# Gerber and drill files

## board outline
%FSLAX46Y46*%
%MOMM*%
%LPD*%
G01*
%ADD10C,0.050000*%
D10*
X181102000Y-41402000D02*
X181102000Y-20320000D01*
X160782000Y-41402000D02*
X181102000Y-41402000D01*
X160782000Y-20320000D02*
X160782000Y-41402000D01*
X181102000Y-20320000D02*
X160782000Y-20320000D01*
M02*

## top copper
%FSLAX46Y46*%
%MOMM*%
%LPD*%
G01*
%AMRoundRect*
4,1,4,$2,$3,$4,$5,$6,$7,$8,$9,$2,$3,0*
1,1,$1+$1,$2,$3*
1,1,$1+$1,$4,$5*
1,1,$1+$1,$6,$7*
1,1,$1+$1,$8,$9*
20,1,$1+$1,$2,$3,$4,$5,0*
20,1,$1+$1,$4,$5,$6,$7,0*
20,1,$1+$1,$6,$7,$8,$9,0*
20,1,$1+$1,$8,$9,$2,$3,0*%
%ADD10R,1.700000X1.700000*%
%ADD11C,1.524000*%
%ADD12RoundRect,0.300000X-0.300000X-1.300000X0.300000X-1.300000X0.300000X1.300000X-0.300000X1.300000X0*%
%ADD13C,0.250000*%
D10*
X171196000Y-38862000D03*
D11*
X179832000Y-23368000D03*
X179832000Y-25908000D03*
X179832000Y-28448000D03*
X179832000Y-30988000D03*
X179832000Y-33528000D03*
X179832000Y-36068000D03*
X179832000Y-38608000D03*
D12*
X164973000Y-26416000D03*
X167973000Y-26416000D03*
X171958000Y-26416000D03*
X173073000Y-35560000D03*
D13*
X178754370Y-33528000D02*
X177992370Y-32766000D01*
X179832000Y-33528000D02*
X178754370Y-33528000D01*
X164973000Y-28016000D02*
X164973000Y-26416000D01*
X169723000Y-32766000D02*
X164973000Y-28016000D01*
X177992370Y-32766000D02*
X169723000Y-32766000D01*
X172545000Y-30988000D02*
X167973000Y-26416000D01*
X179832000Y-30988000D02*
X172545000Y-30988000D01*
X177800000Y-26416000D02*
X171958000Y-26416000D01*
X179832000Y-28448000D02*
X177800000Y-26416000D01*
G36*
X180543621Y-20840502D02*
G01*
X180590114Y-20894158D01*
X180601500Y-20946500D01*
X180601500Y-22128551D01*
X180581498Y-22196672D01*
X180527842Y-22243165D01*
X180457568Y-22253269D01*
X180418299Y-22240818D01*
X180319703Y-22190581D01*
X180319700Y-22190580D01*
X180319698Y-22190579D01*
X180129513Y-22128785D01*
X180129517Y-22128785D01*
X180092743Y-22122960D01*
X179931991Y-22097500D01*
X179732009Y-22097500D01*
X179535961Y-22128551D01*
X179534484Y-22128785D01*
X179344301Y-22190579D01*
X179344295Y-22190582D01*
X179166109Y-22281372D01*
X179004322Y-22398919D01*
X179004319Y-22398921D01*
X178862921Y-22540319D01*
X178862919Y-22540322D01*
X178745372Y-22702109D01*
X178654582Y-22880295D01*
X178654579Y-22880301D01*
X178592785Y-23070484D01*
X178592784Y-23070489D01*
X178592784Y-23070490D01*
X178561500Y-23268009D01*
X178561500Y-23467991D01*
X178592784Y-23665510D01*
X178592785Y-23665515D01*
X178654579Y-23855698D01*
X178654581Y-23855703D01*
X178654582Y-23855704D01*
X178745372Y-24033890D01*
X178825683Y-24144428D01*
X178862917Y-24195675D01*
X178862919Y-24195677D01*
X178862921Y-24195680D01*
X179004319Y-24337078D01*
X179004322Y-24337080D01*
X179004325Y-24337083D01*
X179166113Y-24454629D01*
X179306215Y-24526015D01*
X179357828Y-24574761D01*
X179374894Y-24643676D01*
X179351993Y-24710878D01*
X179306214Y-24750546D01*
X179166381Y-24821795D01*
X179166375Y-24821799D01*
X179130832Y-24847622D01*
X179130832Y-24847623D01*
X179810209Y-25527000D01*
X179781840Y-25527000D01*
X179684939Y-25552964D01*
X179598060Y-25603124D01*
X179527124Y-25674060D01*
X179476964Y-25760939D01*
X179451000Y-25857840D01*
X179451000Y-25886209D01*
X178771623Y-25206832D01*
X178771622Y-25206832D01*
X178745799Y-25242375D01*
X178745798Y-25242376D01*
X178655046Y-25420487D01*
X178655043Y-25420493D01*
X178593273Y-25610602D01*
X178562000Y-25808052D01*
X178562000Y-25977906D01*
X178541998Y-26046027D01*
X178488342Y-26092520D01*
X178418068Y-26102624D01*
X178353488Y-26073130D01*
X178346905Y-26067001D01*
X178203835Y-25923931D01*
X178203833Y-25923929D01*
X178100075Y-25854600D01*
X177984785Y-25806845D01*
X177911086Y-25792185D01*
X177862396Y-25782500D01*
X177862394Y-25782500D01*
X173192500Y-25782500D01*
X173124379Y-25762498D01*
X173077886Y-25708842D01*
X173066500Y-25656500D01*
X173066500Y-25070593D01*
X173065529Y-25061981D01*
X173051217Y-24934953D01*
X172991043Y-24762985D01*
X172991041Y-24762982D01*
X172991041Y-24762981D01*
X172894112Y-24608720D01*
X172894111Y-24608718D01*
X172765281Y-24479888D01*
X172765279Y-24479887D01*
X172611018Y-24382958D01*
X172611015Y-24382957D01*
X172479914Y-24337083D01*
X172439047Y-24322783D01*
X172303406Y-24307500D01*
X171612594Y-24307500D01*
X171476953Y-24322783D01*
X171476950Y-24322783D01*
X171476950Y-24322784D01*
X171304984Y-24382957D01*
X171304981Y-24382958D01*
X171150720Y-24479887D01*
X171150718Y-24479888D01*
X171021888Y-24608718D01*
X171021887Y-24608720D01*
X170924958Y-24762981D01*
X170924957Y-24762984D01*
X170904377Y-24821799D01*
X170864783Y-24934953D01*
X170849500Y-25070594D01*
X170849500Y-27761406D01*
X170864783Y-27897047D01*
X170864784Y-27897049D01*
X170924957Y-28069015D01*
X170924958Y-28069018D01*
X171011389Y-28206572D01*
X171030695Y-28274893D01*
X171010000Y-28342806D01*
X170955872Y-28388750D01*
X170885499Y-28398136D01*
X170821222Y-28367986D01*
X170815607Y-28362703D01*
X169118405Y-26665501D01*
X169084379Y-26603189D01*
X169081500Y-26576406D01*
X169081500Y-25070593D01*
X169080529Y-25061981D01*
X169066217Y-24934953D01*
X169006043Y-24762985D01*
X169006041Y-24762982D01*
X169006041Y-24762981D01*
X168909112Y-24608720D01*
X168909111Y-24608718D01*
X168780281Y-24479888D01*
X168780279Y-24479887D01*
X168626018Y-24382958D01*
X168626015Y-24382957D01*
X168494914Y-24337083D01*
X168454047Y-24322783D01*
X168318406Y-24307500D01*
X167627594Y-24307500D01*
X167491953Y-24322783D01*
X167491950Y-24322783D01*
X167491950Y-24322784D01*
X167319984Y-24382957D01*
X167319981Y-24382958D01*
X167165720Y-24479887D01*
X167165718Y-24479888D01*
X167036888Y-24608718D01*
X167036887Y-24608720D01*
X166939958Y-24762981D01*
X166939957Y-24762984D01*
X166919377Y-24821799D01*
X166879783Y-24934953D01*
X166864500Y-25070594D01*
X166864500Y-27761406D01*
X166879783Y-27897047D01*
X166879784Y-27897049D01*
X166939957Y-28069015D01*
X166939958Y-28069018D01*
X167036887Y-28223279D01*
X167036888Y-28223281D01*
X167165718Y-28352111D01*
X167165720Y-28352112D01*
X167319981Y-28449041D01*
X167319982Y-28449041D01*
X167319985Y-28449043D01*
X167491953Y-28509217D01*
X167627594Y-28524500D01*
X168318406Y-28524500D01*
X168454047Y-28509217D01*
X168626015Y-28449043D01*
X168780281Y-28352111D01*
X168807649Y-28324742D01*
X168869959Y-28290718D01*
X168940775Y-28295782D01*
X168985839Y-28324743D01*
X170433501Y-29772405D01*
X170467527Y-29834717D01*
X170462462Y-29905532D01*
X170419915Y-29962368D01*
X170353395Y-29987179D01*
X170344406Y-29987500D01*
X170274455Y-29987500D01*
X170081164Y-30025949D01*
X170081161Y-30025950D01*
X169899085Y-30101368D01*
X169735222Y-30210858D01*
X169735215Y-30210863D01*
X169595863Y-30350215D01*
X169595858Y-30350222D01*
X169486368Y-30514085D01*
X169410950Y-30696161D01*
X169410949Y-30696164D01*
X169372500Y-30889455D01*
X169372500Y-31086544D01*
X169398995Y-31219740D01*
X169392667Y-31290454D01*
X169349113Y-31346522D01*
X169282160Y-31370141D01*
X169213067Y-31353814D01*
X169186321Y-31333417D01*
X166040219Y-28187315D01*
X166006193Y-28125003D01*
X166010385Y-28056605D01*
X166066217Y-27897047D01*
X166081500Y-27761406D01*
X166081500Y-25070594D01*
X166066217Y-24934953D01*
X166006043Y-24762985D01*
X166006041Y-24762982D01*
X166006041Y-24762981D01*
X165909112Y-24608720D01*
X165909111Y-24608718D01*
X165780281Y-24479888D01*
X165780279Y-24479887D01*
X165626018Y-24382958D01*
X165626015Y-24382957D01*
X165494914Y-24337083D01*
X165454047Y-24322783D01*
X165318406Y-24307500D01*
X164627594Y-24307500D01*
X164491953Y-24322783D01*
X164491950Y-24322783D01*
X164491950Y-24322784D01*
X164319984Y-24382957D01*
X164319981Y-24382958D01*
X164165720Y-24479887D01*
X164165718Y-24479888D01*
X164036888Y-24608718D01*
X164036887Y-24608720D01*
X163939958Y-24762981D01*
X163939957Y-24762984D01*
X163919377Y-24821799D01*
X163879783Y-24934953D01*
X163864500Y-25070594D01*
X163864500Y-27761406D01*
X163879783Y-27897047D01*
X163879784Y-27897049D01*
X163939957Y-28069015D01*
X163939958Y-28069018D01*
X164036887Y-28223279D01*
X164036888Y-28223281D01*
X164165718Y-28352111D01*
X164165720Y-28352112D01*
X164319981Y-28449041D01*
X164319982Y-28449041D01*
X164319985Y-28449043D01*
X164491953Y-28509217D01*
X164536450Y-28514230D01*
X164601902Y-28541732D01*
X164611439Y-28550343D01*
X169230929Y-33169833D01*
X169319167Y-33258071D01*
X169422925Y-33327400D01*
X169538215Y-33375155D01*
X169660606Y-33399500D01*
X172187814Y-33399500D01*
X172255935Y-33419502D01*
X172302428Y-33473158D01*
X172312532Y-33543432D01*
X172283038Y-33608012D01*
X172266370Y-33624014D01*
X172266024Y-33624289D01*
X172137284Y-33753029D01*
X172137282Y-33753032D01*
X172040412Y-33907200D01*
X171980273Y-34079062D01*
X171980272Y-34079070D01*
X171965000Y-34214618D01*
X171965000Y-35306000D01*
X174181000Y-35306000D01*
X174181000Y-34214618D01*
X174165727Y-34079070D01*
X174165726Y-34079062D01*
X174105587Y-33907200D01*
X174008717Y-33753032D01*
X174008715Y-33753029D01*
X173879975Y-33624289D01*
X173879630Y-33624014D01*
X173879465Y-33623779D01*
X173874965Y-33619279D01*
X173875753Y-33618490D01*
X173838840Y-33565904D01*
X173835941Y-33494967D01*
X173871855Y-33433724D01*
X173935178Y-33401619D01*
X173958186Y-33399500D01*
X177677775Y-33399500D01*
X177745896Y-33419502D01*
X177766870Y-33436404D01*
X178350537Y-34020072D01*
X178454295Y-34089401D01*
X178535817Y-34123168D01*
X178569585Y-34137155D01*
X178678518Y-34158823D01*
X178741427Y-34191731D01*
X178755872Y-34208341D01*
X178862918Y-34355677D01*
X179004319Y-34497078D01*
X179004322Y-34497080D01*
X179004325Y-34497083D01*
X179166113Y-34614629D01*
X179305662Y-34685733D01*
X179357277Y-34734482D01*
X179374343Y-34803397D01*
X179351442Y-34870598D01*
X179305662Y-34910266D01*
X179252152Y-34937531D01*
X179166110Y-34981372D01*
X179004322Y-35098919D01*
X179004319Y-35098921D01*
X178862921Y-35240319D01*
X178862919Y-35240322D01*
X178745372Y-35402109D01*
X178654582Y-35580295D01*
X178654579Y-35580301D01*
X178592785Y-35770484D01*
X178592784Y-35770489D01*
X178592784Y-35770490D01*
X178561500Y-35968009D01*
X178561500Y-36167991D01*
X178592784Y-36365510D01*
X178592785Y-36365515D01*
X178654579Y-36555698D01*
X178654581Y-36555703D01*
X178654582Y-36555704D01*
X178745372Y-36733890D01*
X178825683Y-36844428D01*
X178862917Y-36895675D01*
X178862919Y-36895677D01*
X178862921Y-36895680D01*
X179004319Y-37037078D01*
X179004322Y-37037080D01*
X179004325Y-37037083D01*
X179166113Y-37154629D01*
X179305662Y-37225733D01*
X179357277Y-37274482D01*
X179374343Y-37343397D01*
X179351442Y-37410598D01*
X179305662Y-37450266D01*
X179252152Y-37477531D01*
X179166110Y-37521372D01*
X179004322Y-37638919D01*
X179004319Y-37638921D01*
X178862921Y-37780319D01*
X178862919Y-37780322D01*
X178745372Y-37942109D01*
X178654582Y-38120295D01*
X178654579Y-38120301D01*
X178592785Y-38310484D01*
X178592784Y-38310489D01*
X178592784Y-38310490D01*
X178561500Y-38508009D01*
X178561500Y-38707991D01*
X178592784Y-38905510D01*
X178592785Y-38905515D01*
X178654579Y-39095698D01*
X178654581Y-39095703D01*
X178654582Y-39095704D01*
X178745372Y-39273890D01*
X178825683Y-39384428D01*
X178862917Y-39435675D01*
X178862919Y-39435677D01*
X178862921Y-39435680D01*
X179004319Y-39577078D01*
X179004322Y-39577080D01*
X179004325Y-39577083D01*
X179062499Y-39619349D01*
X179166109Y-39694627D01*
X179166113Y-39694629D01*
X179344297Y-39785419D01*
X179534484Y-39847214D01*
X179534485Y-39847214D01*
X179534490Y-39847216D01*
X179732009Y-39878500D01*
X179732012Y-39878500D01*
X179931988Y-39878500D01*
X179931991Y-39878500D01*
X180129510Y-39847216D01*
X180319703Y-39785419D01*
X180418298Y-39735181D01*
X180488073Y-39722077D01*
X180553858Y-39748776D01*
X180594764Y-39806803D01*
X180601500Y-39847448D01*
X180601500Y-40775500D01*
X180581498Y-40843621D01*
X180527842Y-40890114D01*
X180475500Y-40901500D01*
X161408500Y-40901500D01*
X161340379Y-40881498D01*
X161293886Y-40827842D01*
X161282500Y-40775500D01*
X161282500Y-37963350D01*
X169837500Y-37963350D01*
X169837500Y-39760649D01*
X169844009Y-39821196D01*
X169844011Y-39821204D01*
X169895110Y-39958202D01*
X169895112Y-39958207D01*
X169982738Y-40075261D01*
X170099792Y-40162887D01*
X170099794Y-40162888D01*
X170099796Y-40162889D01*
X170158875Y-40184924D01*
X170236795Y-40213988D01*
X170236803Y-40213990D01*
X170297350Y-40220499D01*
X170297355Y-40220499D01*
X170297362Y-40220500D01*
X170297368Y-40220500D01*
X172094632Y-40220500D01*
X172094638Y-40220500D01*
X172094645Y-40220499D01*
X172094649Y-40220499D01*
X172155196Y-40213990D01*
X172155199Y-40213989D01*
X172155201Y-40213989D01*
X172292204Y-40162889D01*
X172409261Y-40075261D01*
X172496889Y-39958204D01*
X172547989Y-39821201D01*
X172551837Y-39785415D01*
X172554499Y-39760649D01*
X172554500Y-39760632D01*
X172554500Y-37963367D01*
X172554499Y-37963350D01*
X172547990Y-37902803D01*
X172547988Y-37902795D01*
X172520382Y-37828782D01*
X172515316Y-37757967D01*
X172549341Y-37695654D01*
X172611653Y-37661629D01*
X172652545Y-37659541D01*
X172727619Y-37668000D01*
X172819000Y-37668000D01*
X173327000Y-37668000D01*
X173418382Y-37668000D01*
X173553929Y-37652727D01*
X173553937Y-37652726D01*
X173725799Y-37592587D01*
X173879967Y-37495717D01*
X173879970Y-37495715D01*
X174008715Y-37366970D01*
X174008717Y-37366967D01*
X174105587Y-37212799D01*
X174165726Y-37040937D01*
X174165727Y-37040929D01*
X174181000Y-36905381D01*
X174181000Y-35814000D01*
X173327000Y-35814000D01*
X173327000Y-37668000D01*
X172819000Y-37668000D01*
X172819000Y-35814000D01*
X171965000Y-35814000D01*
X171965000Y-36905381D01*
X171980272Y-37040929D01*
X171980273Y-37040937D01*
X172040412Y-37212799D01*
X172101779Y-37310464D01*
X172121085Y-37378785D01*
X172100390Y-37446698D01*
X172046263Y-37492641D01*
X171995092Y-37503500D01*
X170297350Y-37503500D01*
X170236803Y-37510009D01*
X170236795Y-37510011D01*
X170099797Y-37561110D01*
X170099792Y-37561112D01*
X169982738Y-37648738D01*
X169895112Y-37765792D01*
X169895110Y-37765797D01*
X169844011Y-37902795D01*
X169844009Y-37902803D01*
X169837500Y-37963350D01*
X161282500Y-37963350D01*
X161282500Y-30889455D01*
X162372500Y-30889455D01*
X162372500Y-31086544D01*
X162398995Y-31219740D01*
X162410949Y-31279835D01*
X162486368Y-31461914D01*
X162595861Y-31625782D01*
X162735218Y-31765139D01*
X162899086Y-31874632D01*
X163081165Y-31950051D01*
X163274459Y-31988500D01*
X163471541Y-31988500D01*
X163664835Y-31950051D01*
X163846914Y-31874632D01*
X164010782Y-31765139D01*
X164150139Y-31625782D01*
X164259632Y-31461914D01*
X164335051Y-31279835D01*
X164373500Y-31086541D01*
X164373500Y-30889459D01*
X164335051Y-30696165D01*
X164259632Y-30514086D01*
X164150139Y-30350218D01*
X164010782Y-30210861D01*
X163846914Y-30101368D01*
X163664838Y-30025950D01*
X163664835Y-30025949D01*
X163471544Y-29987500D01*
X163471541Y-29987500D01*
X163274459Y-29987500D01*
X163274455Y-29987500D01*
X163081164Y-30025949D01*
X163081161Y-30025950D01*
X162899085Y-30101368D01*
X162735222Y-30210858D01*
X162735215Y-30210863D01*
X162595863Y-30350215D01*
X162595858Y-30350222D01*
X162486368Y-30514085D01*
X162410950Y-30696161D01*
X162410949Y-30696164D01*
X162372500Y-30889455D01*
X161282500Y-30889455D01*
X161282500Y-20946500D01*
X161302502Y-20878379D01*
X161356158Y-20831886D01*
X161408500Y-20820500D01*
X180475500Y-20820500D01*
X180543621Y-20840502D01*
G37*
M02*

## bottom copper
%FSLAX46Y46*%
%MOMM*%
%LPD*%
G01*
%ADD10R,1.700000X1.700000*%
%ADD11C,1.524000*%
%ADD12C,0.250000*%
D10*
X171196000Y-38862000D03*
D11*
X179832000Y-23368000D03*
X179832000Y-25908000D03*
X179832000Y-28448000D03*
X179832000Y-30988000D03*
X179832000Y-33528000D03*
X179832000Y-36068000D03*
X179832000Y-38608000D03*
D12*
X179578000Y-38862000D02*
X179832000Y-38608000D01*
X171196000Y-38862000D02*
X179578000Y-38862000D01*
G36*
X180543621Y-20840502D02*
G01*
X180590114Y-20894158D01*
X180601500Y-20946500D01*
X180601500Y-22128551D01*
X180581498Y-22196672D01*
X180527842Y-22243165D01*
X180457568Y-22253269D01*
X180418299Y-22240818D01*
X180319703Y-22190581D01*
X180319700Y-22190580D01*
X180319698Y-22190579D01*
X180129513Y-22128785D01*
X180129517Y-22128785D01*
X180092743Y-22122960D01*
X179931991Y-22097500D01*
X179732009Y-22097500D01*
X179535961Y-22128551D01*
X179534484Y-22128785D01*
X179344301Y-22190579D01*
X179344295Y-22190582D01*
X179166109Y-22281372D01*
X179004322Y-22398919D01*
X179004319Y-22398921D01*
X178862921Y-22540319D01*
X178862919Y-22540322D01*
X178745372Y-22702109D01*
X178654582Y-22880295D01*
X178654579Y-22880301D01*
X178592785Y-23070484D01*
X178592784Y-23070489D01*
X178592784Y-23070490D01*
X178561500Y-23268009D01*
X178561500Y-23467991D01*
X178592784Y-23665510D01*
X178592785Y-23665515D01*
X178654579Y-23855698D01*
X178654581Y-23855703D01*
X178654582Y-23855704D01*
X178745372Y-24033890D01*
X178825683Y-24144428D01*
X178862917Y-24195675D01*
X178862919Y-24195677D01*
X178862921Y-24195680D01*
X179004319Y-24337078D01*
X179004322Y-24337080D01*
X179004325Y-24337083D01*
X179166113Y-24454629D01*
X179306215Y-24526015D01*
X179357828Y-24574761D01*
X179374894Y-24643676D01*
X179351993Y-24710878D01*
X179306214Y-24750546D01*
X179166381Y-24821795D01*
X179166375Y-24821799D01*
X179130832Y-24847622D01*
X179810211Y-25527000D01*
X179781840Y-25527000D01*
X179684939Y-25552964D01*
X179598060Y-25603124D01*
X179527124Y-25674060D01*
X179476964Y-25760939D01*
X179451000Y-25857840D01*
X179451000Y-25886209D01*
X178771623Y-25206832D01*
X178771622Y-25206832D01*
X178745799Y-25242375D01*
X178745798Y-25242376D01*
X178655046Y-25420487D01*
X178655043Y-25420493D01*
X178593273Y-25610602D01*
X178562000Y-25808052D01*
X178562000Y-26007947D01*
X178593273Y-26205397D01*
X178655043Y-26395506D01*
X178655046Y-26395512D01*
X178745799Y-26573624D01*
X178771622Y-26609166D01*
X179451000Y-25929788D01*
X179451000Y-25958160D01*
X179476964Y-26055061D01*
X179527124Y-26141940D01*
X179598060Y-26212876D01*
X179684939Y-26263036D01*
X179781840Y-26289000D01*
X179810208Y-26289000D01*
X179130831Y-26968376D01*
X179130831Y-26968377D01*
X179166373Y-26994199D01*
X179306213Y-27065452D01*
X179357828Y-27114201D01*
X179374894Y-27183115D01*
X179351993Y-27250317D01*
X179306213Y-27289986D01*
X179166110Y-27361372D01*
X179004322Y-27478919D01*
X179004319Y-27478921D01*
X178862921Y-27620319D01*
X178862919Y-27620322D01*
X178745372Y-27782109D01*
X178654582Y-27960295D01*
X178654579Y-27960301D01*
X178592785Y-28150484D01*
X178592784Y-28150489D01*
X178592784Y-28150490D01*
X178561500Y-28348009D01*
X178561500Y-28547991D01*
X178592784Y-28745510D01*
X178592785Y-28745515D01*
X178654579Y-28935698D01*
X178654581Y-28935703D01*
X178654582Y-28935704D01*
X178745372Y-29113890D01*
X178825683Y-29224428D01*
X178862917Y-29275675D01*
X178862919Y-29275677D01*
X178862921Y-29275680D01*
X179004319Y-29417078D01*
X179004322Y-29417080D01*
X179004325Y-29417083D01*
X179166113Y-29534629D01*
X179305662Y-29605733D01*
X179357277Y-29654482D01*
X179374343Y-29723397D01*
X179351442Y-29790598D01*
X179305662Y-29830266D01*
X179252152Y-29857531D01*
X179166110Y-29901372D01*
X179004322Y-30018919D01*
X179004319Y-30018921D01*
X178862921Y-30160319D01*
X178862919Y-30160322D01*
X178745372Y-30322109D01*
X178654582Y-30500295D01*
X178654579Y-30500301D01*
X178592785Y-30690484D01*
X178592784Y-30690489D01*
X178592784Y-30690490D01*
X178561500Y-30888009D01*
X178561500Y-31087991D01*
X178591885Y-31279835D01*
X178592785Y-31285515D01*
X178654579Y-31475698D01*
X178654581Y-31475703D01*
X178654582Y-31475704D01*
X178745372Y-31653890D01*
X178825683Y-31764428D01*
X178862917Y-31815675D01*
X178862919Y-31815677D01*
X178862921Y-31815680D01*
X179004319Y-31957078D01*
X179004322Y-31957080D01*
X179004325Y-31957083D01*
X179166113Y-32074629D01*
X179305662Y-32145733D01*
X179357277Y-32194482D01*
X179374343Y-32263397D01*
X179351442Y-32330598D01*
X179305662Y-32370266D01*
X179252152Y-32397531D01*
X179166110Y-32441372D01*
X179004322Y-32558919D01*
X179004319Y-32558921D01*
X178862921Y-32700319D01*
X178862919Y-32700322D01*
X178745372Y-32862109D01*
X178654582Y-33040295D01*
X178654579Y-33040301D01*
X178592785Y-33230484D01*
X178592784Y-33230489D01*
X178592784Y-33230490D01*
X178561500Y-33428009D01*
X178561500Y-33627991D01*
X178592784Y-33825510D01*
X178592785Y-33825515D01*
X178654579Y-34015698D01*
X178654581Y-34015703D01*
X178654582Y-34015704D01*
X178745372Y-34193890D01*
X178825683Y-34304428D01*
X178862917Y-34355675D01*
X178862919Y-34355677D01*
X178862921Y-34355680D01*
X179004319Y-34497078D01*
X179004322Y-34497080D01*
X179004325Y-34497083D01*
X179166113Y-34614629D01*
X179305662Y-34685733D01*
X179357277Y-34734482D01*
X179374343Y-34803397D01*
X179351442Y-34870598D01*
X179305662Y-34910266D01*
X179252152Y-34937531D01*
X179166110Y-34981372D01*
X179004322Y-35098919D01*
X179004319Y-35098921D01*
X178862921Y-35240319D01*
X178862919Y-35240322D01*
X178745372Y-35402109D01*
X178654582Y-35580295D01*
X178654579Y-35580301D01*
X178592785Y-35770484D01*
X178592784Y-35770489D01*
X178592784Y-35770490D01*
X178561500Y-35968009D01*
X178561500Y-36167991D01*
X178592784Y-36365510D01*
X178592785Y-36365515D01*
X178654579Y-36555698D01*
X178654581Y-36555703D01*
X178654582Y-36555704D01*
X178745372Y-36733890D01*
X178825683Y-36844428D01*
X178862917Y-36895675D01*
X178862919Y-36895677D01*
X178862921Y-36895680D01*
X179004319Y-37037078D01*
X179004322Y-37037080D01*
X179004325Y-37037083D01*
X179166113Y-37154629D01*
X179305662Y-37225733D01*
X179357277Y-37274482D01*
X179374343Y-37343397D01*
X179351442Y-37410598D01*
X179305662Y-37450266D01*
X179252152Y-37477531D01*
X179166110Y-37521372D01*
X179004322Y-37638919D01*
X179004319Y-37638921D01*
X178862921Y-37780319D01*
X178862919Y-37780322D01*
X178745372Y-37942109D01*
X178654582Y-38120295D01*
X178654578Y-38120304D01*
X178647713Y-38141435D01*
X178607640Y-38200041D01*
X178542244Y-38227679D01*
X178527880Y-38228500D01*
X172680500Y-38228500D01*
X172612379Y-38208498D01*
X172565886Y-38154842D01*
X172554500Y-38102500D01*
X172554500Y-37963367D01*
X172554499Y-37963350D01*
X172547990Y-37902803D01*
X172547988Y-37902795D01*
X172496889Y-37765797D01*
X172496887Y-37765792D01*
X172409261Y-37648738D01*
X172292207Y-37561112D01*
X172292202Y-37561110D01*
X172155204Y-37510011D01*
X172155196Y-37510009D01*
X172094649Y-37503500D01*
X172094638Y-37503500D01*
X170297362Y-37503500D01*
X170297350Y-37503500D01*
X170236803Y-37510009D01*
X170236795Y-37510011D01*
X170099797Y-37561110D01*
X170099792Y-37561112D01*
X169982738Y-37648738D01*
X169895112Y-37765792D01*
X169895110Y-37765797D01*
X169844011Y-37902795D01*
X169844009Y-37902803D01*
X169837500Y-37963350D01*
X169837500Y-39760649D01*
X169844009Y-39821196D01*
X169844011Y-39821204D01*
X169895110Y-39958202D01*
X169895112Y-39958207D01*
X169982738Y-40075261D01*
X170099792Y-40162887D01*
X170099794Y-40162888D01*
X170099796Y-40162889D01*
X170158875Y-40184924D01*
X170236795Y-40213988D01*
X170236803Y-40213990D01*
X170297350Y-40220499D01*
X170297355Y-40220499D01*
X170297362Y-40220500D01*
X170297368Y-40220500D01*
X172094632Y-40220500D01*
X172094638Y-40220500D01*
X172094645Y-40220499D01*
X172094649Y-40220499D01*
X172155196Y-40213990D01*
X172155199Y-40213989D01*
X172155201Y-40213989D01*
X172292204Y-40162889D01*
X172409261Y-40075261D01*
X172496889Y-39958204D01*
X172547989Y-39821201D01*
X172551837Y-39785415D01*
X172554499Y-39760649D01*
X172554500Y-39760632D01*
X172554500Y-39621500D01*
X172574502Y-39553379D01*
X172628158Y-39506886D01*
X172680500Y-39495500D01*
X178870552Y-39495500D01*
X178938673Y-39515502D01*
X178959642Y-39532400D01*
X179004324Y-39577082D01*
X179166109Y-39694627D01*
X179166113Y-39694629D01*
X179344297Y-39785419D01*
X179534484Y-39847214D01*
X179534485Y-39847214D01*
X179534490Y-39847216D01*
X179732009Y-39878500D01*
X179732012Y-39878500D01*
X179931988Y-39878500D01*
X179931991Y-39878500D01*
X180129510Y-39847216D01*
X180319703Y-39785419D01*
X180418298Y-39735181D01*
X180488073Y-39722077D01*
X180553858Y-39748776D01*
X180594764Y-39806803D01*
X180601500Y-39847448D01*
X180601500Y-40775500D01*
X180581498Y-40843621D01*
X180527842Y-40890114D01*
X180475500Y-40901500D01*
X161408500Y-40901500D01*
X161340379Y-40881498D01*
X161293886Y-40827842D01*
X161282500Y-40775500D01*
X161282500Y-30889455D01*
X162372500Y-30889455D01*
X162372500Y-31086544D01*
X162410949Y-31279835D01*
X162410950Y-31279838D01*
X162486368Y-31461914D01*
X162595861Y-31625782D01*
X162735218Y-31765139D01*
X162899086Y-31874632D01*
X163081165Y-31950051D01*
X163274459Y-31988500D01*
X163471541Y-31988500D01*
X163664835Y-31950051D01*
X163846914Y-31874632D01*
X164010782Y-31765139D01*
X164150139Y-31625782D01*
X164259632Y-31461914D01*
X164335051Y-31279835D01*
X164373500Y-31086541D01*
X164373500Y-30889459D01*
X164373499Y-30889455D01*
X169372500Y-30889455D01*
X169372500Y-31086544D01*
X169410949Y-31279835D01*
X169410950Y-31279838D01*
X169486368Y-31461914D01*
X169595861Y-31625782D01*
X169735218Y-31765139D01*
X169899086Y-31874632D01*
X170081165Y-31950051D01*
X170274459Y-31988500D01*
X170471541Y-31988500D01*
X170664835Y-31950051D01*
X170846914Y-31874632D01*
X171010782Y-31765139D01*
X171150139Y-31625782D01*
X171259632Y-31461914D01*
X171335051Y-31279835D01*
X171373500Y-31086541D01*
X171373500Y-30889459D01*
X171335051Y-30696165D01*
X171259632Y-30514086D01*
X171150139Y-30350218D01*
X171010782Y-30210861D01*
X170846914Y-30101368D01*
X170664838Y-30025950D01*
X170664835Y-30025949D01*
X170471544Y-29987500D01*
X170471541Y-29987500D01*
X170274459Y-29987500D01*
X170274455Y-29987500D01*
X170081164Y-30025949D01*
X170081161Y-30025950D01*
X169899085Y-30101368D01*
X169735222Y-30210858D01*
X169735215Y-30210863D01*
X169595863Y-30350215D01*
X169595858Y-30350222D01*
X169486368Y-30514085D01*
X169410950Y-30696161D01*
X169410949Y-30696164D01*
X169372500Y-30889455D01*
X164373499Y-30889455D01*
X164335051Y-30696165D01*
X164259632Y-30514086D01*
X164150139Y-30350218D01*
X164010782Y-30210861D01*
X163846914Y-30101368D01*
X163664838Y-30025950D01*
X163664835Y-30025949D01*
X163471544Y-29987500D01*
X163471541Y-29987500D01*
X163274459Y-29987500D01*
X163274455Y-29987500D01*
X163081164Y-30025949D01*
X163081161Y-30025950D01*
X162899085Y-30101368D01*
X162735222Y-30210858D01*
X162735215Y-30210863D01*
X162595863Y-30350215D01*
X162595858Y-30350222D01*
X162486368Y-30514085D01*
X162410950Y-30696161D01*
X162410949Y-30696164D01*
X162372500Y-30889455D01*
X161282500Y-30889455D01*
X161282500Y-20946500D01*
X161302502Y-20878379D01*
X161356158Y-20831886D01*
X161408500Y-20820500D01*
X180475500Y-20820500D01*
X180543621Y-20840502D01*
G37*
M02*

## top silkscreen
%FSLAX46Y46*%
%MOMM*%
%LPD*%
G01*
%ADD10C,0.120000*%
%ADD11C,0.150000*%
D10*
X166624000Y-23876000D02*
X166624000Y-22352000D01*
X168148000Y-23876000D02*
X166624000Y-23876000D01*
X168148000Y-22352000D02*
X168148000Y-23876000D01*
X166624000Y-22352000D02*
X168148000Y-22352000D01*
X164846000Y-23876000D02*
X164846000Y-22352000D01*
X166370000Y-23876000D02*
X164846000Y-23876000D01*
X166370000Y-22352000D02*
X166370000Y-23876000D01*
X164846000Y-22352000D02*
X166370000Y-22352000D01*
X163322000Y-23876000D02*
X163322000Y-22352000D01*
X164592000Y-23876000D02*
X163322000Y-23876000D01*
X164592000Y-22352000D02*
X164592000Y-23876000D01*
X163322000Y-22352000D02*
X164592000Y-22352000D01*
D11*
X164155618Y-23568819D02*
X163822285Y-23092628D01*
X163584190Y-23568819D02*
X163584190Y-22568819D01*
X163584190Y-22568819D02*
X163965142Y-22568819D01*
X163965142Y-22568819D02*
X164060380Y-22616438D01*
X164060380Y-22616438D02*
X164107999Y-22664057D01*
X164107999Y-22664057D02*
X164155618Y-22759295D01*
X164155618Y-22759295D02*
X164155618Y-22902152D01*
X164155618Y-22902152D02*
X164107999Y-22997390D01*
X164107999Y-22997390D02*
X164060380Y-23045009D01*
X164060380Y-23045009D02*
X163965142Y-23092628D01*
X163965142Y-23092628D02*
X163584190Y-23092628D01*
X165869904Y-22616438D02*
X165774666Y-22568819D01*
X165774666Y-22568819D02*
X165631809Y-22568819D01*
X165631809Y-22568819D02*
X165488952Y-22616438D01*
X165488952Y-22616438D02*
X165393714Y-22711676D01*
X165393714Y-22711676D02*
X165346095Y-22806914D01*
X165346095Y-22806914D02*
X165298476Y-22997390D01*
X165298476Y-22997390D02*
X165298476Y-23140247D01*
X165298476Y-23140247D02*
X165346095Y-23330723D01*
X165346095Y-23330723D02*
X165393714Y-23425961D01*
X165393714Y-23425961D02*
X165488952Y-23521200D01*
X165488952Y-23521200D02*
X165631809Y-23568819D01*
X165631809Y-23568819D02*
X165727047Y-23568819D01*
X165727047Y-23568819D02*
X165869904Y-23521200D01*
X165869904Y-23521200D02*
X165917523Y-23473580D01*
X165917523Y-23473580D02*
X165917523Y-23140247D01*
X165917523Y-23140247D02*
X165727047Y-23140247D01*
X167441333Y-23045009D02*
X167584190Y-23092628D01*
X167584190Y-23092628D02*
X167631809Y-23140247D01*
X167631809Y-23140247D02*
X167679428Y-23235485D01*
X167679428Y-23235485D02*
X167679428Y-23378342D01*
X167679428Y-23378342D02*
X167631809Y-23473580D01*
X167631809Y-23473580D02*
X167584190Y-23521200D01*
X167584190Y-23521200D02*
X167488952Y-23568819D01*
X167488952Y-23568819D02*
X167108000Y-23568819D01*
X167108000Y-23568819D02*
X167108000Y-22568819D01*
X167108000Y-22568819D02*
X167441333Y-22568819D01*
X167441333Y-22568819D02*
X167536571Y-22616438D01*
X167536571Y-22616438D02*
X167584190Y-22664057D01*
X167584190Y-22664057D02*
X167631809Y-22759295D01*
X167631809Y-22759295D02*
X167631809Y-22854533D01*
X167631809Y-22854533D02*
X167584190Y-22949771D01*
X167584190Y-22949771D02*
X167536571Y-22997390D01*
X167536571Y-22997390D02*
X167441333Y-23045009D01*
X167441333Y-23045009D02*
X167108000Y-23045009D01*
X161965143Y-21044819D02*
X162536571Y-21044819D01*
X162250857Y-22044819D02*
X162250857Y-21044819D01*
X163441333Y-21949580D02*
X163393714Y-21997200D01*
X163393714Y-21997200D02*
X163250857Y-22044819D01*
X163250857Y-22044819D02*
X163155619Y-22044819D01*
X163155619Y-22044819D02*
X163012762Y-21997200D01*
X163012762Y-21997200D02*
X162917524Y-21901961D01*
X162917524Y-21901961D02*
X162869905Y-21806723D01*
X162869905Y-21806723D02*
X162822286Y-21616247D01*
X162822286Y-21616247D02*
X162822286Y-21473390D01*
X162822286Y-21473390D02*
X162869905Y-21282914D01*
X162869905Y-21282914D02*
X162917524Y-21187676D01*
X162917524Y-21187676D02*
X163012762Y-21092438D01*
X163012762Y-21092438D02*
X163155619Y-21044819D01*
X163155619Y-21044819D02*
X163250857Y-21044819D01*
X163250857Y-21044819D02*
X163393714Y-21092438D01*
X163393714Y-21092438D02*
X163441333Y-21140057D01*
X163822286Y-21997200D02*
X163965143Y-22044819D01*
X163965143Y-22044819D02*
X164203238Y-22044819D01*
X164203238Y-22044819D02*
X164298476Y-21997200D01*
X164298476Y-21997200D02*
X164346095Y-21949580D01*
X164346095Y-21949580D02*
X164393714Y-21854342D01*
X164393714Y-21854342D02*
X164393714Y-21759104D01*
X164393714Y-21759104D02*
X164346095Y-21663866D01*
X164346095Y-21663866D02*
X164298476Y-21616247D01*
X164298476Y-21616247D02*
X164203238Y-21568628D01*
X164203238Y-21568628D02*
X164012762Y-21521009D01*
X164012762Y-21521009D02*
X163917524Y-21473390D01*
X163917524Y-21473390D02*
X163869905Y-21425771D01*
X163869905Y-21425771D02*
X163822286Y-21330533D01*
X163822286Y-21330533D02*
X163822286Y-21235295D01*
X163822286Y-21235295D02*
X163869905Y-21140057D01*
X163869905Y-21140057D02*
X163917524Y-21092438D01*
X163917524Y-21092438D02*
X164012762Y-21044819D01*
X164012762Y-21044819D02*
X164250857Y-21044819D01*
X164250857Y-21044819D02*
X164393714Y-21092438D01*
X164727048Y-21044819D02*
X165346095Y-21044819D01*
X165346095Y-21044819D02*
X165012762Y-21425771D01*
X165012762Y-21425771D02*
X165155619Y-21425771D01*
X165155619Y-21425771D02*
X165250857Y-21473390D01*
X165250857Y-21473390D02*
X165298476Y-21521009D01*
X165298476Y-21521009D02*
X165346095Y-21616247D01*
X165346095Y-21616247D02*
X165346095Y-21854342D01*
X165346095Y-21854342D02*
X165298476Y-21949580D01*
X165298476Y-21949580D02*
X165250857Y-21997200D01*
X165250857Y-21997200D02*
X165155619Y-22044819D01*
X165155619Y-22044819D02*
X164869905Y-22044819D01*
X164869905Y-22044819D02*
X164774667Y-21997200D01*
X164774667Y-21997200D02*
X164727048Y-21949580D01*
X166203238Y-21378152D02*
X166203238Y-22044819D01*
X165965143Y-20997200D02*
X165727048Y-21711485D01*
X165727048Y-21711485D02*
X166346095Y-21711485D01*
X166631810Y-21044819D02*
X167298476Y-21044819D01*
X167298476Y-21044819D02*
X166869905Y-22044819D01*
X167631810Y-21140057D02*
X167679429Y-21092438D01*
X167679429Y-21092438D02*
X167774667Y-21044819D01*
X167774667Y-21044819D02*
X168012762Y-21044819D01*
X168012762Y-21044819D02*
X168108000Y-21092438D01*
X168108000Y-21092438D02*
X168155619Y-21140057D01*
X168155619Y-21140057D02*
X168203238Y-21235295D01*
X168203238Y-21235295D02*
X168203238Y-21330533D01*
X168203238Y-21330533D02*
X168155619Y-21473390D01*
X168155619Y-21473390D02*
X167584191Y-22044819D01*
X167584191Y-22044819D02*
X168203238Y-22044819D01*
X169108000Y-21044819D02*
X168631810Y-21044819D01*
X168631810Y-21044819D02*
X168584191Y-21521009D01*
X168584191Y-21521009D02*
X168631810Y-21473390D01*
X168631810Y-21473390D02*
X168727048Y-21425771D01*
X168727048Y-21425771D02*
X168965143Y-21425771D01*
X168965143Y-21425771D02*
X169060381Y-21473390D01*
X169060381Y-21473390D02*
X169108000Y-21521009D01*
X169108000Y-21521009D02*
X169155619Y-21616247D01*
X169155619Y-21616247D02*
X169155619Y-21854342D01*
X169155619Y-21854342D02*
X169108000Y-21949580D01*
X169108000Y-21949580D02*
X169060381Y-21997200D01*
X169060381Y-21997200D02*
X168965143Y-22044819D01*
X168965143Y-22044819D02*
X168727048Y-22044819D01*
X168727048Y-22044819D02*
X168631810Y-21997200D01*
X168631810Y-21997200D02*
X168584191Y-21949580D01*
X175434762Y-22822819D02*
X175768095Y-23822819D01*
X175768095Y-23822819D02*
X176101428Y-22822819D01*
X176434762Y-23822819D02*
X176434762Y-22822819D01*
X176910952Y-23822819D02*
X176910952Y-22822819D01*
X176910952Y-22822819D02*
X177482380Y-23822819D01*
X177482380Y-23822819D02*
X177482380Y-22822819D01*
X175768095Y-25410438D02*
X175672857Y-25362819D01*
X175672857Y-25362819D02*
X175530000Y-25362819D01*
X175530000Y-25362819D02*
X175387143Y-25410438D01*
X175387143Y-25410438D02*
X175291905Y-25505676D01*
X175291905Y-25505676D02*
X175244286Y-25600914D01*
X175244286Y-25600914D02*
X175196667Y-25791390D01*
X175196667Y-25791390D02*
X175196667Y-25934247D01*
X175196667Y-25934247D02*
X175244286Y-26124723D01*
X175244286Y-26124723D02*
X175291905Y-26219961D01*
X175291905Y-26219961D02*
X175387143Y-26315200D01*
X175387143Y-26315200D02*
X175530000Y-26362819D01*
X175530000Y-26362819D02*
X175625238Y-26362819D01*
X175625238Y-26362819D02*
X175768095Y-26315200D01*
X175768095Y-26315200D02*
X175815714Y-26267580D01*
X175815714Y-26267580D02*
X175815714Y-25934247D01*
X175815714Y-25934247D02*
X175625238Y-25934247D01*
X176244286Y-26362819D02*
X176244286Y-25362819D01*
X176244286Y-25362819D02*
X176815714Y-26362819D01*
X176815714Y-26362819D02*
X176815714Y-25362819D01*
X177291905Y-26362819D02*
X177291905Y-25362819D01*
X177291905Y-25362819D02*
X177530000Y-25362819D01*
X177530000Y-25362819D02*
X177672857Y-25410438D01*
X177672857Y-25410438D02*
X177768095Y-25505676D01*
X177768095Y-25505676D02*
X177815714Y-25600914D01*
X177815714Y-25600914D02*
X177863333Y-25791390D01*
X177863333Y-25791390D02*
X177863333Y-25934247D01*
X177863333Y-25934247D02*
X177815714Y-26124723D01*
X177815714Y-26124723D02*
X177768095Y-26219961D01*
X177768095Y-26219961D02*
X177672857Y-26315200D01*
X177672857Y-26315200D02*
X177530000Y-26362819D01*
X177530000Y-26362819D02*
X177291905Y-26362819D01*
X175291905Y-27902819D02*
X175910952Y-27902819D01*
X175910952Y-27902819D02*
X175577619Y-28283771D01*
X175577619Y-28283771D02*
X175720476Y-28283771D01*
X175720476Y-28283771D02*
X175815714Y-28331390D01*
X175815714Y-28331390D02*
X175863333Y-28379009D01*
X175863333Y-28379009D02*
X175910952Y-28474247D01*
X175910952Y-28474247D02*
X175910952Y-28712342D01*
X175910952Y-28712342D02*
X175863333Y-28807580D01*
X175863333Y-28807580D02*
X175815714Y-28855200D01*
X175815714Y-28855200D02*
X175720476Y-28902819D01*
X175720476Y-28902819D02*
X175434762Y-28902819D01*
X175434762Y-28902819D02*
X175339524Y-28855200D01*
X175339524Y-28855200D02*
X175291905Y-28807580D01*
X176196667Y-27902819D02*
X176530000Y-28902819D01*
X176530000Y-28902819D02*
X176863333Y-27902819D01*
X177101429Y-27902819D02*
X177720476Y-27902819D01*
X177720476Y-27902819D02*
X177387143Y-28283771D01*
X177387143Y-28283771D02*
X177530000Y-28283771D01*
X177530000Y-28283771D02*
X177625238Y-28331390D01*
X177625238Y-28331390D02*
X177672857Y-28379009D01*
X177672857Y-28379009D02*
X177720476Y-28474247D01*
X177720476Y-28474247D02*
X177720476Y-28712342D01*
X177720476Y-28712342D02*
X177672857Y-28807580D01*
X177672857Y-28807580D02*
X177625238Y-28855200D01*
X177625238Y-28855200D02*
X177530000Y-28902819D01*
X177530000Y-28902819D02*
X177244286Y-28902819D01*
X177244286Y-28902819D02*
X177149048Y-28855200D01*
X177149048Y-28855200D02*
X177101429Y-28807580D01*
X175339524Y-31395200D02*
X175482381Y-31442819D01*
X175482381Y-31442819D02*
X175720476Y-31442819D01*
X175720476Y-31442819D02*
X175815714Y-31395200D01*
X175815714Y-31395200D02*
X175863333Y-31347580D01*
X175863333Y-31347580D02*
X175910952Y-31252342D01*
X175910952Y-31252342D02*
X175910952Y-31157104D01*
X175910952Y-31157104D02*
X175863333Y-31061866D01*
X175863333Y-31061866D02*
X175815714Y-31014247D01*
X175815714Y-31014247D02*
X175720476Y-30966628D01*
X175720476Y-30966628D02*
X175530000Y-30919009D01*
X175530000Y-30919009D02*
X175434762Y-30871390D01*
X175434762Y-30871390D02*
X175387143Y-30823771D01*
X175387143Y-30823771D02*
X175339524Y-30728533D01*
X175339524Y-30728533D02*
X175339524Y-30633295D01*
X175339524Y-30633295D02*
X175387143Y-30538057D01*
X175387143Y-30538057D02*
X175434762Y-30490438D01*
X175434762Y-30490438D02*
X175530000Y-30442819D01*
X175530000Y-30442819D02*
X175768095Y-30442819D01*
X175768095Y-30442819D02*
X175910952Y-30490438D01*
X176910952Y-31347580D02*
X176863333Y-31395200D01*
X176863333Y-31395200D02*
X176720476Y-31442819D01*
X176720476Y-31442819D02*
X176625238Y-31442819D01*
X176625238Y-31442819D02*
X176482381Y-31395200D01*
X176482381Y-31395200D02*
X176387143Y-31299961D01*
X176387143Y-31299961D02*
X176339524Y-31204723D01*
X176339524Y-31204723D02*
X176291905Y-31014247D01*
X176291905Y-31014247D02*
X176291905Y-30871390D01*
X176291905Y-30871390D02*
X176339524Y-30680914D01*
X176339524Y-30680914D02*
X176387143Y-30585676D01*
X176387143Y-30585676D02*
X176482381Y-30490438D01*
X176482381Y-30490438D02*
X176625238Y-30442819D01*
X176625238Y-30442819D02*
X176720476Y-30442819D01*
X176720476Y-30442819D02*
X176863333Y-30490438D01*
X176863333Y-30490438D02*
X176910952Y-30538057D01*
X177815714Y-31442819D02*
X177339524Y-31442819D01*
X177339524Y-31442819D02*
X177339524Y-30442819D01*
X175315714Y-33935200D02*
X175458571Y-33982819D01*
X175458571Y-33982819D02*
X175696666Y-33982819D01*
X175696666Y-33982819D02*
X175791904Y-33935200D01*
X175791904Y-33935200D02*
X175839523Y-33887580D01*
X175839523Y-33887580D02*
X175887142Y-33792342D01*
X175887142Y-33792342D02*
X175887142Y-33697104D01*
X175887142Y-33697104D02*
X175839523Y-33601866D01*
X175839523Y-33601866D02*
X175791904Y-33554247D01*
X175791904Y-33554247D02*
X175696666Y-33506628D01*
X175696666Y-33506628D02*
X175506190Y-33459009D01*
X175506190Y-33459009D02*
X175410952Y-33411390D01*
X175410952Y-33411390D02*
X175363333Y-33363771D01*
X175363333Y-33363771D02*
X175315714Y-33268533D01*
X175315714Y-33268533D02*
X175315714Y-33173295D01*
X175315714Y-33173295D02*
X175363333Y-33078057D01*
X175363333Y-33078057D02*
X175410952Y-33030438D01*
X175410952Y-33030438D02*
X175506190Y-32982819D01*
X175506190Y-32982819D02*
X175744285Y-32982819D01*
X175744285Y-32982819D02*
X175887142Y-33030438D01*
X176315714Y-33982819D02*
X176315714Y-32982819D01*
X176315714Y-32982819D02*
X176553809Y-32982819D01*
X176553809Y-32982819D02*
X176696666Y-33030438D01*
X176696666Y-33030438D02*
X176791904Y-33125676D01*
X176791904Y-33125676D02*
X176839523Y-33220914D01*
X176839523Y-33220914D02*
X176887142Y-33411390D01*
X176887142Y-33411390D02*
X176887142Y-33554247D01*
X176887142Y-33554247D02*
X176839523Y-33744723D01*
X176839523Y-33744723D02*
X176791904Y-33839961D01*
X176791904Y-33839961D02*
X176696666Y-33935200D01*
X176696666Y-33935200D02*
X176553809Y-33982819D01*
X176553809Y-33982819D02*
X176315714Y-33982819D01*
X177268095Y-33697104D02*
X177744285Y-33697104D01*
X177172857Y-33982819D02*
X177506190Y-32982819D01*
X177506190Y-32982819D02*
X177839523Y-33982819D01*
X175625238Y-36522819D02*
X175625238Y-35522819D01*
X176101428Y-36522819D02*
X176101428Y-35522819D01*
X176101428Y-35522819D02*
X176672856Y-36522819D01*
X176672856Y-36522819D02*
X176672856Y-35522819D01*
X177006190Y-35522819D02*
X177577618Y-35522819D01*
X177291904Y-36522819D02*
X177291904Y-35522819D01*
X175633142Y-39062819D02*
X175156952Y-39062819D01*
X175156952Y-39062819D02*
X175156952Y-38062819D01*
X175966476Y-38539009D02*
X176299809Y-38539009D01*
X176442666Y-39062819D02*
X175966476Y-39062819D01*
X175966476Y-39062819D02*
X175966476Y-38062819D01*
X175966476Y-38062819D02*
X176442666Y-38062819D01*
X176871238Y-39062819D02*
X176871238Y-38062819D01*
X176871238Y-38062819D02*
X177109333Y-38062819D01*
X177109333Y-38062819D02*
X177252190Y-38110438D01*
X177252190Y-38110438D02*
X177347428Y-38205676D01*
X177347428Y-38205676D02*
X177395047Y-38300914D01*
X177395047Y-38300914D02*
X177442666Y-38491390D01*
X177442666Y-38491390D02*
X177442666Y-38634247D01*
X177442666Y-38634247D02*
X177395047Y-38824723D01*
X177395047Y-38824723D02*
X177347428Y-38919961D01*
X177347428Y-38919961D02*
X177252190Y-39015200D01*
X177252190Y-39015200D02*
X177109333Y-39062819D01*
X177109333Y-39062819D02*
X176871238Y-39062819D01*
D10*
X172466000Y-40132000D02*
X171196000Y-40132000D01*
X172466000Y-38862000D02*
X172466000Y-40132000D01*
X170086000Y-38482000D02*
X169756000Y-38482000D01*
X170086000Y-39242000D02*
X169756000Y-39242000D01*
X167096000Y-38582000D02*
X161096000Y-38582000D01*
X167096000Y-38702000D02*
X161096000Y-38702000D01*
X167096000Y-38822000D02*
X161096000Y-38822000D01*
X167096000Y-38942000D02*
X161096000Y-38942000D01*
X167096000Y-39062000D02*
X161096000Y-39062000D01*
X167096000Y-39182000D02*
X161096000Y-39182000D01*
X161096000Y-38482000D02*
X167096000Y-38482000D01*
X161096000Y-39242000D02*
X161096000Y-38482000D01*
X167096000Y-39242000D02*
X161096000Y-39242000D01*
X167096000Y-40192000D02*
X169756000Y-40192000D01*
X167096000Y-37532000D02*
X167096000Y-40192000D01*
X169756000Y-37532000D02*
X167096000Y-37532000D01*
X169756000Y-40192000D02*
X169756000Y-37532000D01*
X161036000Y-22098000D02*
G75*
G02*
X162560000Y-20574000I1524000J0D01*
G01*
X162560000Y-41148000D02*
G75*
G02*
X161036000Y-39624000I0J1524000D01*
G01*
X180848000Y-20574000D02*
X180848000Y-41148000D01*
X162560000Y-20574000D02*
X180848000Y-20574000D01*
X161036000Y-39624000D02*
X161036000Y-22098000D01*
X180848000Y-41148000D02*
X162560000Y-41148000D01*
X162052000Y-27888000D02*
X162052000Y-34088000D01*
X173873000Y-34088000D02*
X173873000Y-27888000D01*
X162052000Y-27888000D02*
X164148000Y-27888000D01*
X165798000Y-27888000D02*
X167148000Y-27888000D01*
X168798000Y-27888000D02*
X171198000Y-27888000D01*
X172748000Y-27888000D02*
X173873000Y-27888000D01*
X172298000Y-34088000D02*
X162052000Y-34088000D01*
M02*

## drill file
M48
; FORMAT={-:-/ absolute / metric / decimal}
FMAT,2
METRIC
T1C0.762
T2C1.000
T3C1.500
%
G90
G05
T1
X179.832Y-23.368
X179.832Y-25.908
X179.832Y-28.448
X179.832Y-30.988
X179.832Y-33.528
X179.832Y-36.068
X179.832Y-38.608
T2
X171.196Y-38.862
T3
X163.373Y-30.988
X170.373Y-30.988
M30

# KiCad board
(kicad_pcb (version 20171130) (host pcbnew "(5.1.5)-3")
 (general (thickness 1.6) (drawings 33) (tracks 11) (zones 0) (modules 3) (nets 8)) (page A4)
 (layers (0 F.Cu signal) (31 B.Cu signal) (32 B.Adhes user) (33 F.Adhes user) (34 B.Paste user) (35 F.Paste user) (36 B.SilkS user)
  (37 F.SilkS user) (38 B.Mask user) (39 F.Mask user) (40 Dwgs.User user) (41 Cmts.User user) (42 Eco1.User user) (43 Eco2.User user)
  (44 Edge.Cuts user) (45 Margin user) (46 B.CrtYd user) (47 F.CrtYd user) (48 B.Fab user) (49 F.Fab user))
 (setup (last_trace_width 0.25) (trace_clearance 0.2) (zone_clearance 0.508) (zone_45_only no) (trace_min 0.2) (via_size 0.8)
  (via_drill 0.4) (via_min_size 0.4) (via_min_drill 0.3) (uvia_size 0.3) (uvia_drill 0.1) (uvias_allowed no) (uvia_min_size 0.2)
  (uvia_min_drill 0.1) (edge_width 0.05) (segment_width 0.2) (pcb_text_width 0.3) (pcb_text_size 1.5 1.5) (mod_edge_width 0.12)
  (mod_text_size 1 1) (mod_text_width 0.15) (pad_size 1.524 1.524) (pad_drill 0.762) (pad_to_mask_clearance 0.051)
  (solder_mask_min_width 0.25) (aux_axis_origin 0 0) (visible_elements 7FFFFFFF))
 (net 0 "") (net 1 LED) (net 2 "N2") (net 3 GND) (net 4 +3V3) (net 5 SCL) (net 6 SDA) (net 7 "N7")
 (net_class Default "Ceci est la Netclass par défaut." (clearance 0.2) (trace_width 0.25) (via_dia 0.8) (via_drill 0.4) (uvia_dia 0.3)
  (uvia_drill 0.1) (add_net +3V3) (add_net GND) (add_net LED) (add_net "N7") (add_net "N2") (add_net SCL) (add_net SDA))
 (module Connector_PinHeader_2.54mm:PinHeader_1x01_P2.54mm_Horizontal (layer F.Cu) (at 171.196 38.862 180)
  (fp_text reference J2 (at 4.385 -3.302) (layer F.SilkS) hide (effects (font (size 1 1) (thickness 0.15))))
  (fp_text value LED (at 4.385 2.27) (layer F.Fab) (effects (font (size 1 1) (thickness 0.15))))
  (fp_line (start -1.27 -1.27) (end 0 -1.27) (layer F.SilkS) (width 0.12))
  (fp_line (start -1.27 0) (end -1.27 -1.27) (layer F.SilkS) (width 0.12))
  (fp_line (start 1.11 0.38) (end 1.44 0.38) (layer F.SilkS) (width 0.12))
  (fp_line (start 1.11 -0.38) (end 1.44 -0.38) (layer F.SilkS) (width 0.12))
  (fp_line (start 4.1 0.28) (end 10.1 0.28) (layer F.SilkS) (width 0.12))
  (fp_line (start 4.1 0.16) (end 10.1 0.16) (layer F.SilkS) (width 0.12))
  (fp_line (start 4.1 0.04) (end 10.1 0.04) (layer F.SilkS) (width 0.12))
  (fp_line (start 4.1 -0.08) (end 10.1 -0.08) (layer F.SilkS) (width 0.12))
  (fp_line (start 4.1 -0.2) (end 10.1 -0.2) (layer F.SilkS) (width 0.12))
  (fp_line (start 4.1 -0.32) (end 10.1 -0.32) (layer F.SilkS) (width 0.12))
  (fp_line (start 10.1 0.38) (end 4.1 0.38) (layer F.SilkS) (width 0.12))
  (fp_line (start 10.1 -0.38) (end 10.1 0.38) (layer F.SilkS) (width 0.12))
  (fp_line (start 4.1 -0.38) (end 10.1 -0.38) (layer F.SilkS) (width 0.12))
  (fp_line (start 4.1 -1.33) (end 1.44 -1.33) (layer F.SilkS) (width 0.12))
  (fp_line (start 4.1 1.33) (end 4.1 -1.33) (layer F.SilkS) (width 0.12))
  (fp_line (start 1.44 1.33) (end 4.1 1.33) (layer F.SilkS) (width 0.12))
  (fp_line (start 1.44 -1.33) (end 1.44 1.33) (layer F.SilkS) (width 0.12))
  (pad 1 thru_hole rect (at 0 0 180) (size 1.7 1.7) (drill 1) (layers *.Cu *.Mask) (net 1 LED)))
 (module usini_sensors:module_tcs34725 (layer F.Cu) (at 177.292 23.368 180)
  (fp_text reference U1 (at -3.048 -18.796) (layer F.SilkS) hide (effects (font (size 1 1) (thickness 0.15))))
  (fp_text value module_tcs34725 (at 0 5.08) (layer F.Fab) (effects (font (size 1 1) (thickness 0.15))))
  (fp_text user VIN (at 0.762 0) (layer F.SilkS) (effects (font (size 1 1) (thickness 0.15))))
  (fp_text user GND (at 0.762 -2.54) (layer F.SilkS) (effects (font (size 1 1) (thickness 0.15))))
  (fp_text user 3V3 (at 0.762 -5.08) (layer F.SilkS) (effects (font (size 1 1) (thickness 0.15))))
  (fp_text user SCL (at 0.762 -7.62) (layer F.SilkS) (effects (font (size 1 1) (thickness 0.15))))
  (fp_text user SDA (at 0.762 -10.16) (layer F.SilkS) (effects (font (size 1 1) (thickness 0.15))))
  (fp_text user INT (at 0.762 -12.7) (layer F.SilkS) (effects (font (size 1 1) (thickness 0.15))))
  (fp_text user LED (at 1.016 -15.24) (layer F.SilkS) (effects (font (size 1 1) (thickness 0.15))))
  (fp_arc (start 14.732 1.27) (end 14.732 2.794) (angle -90) (layer F.SilkS) (width 0.12))
  (fp_arc (start 14.732 -16.256) (end 16.256 -16.256) (angle -90) (layer F.SilkS) (width 0.12))
  (fp_line (start -3.556 2.794) (end -3.556 -17.78) (layer F.SilkS) (width 0.12))
  (fp_line (start 14.732 2.794) (end -3.556 2.794) (layer F.SilkS) (width 0.12))
  (fp_line (start 16.256 -16.256) (end 16.256 1.27) (layer F.SilkS) (width 0.12))
  (fp_line (start -3.556 -17.78) (end 14.732 -17.78) (layer F.SilkS) (width 0.12))
  (pad 7 thru_hole circle (at -2.54 0 180) (size 1.524 1.524) (drill 0.762) (layers *.Cu *.Mask) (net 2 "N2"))
  (pad 6 thru_hole circle (at -2.54 -2.54 180) (size 1.524 1.524) (drill 0.762) (layers *.Cu *.Mask) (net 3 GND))
  (pad 5 thru_hole circle (at -2.54 -5.08 180) (size 1.524 1.524) (drill 0.762) (layers *.Cu *.Mask) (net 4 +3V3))
  (pad 4 thru_hole circle (at -2.54 -7.62 180) (size 1.524 1.524) (drill 0.762) (layers *.Cu *.Mask) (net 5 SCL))
  (pad 3 thru_hole circle (at -2.54 -10.16 180) (size 1.524 1.524) (drill 0.762) (layers *.Cu *.Mask) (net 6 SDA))
  (pad 2 thru_hole circle (at -2.54 -12.7 180) (size 1.524 1.524) (drill 0.762) (layers *.Cu *.Mask) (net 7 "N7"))
  (pad 1 thru_hole circle (at -2.54 -15.24 180) (size 1.524 1.524) (drill 0.762) (layers *.Cu *.Mask) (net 1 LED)))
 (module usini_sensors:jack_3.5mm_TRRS (layer F.Cu) (at 168.148 30.988)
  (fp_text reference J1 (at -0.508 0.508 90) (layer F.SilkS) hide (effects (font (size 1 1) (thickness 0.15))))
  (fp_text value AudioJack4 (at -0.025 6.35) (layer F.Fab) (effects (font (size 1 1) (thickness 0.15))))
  (fp_line (start -6.096 -3.1) (end -6.096 3.1) (layer F.SilkS) (width 0.12))
  (fp_line (start 5.725 3.1) (end 5.725 -3.1) (layer F.SilkS) (width 0.12))
  (fp_line (start -6.096 -3.1) (end -4 -3.1) (layer F.SilkS) (width 0.12))
  (fp_line (start -2.35 -3.1) (end -1 -3.1) (layer F.SilkS) (width 0.12))
  (fp_line (start 0.65 -3.1) (end 3.05 -3.1) (layer F.SilkS) (width 0.12))
  (fp_line (start 4.6 -3.1) (end 5.725 -3.1) (layer F.SilkS) (width 0.12))
  (fp_line (start 4.15 3.1) (end -6.096 3.1) (layer F.SilkS) (width 0.12))
  (pad "" np_thru_hole circle (at 2.225 0) (size 1.5 1.5) (drill 1.5) (layers *.Cu *.Mask))
  (pad "" np_thru_hole circle (at -4.775 0) (size 1.5 1.5) (drill 1.5) (layers *.Cu *.Mask))
  (pad R2 smd roundrect (at -3.175 -4.572) (size 1.2 3.2) (layers F.Cu F.Paste F.Mask) (roundrect_rratio 0.25) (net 6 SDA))
  (pad R1 smd roundrect (at -0.175 -4.572) (size 1.2 3.2) (layers F.Cu F.Paste F.Mask) (roundrect_rratio 0.25) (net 5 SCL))
  (pad T smd roundrect (at 3.81 -4.572) (size 1.2 3.2) (layers F.Cu F.Paste F.Mask) (roundrect_rratio 0.25) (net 4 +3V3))
  (pad S smd roundrect (at 4.925 4.572) (size 1.2 3.2) (layers F.Cu F.Paste F.Mask) (roundrect_rratio 0.25) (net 3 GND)))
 (gr_line (start 166.624 23.876) (end 166.624 22.352) (layer F.SilkS) (width 0.12))
 (gr_line (start 168.148 23.876) (end 166.624 23.876) (layer F.SilkS) (width 0.12))
 (gr_line (start 168.148 22.352) (end 168.148 23.876) (layer F.SilkS) (width 0.12))
 (gr_line (start 166.624 22.352) (end 168.148 22.352) (layer F.SilkS) (width 0.12))
 (gr_line (start 164.846 23.876) (end 164.846 22.352) (layer F.SilkS) (width 0.12))
 (gr_line (start 166.37 23.876) (end 164.846 23.876) (layer F.SilkS) (width 0.12))
 (gr_line (start 166.37 22.352) (end 166.37 23.876) (layer F.SilkS) (width 0.12))
 (gr_line (start 164.846 22.352) (end 166.37 22.352) (layer F.SilkS) (width 0.12))
 (gr_line (start 163.322 23.876) (end 163.322 22.352) (layer F.SilkS) (width 0.12))
 (gr_line (start 164.592 23.876) (end 163.322 23.876) (layer F.SilkS) (width 0.12))
 (gr_line (start 164.592 22.352) (end 164.592 23.876) (layer F.SilkS) (width 0.12))
 (gr_line (start 163.322 22.352) (end 164.592 22.352) (layer F.SilkS) (width 0.12))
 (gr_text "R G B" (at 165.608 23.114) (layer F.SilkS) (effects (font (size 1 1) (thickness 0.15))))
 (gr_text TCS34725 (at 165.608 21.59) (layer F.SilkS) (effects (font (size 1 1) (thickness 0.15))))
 (gr_line (start 181.102 41.402) (end 181.102 20.32) (layer Edge.Cuts) (width 0.05))
 (gr_line (start 160.782 41.402) (end 181.102 41.402) (layer Edge.Cuts) (width 0.05))
 (gr_line (start 160.782 20.32) (end 160.782 41.402) (layer Edge.Cuts) (width 0.05))
 (gr_line (start 181.102 20.32) (end 160.782 20.32) (layer Edge.Cuts) (width 0.05))
 (segment (start 178.75437 33.528) (end 177.99237 32.766) (width 0.25) (layer F.Cu) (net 6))
 (segment (start 179.832 33.528) (end 178.75437 33.528) (width 0.25) (layer F.Cu) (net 6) (status 10))
 (segment (start 164.973 28.016) (end 164.973 26.416) (width 0.25) (layer F.Cu) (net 6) (status 20))
 (segment (start 169.723 32.766) (end 164.973 28.016) (width 0.25) (layer F.Cu) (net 6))
 (segment (start 177.99237 32.766) (end 169.723 32.766) (width 0.25) (layer F.Cu) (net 6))
 (segment (start 172.545 30.988) (end 167.973 26.416) (width 0.25) (layer F.Cu) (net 5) (status 20))
 (segment (start 179.832 30.988) (end 172.545 30.988) (width 0.25) (layer F.Cu) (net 5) (status 10))
 (segment (start 177.8 26.416) (end 171.958 26.416) (width 0.25) (layer F.Cu) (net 4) (status 20))
 (segment (start 179.832 28.448) (end 177.8 26.416) (width 0.25) (layer F.Cu) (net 4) (status 10))
 (segment (start 179.578 38.862) (end 179.832 38.608) (width 0.25) (layer B.Cu) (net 1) (status 30))
 (segment (start 171.196 38.862) (end 179.578 38.862) (width 0.25) (layer B.Cu) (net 1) (status 30))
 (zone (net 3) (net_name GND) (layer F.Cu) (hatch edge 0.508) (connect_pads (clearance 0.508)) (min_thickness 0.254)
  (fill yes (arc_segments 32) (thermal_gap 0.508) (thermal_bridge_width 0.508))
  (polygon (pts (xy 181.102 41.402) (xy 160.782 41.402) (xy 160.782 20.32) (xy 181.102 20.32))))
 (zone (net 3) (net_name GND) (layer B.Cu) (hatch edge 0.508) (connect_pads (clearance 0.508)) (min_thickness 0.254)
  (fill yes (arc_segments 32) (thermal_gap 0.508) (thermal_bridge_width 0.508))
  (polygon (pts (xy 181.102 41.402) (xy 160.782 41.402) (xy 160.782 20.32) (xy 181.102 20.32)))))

